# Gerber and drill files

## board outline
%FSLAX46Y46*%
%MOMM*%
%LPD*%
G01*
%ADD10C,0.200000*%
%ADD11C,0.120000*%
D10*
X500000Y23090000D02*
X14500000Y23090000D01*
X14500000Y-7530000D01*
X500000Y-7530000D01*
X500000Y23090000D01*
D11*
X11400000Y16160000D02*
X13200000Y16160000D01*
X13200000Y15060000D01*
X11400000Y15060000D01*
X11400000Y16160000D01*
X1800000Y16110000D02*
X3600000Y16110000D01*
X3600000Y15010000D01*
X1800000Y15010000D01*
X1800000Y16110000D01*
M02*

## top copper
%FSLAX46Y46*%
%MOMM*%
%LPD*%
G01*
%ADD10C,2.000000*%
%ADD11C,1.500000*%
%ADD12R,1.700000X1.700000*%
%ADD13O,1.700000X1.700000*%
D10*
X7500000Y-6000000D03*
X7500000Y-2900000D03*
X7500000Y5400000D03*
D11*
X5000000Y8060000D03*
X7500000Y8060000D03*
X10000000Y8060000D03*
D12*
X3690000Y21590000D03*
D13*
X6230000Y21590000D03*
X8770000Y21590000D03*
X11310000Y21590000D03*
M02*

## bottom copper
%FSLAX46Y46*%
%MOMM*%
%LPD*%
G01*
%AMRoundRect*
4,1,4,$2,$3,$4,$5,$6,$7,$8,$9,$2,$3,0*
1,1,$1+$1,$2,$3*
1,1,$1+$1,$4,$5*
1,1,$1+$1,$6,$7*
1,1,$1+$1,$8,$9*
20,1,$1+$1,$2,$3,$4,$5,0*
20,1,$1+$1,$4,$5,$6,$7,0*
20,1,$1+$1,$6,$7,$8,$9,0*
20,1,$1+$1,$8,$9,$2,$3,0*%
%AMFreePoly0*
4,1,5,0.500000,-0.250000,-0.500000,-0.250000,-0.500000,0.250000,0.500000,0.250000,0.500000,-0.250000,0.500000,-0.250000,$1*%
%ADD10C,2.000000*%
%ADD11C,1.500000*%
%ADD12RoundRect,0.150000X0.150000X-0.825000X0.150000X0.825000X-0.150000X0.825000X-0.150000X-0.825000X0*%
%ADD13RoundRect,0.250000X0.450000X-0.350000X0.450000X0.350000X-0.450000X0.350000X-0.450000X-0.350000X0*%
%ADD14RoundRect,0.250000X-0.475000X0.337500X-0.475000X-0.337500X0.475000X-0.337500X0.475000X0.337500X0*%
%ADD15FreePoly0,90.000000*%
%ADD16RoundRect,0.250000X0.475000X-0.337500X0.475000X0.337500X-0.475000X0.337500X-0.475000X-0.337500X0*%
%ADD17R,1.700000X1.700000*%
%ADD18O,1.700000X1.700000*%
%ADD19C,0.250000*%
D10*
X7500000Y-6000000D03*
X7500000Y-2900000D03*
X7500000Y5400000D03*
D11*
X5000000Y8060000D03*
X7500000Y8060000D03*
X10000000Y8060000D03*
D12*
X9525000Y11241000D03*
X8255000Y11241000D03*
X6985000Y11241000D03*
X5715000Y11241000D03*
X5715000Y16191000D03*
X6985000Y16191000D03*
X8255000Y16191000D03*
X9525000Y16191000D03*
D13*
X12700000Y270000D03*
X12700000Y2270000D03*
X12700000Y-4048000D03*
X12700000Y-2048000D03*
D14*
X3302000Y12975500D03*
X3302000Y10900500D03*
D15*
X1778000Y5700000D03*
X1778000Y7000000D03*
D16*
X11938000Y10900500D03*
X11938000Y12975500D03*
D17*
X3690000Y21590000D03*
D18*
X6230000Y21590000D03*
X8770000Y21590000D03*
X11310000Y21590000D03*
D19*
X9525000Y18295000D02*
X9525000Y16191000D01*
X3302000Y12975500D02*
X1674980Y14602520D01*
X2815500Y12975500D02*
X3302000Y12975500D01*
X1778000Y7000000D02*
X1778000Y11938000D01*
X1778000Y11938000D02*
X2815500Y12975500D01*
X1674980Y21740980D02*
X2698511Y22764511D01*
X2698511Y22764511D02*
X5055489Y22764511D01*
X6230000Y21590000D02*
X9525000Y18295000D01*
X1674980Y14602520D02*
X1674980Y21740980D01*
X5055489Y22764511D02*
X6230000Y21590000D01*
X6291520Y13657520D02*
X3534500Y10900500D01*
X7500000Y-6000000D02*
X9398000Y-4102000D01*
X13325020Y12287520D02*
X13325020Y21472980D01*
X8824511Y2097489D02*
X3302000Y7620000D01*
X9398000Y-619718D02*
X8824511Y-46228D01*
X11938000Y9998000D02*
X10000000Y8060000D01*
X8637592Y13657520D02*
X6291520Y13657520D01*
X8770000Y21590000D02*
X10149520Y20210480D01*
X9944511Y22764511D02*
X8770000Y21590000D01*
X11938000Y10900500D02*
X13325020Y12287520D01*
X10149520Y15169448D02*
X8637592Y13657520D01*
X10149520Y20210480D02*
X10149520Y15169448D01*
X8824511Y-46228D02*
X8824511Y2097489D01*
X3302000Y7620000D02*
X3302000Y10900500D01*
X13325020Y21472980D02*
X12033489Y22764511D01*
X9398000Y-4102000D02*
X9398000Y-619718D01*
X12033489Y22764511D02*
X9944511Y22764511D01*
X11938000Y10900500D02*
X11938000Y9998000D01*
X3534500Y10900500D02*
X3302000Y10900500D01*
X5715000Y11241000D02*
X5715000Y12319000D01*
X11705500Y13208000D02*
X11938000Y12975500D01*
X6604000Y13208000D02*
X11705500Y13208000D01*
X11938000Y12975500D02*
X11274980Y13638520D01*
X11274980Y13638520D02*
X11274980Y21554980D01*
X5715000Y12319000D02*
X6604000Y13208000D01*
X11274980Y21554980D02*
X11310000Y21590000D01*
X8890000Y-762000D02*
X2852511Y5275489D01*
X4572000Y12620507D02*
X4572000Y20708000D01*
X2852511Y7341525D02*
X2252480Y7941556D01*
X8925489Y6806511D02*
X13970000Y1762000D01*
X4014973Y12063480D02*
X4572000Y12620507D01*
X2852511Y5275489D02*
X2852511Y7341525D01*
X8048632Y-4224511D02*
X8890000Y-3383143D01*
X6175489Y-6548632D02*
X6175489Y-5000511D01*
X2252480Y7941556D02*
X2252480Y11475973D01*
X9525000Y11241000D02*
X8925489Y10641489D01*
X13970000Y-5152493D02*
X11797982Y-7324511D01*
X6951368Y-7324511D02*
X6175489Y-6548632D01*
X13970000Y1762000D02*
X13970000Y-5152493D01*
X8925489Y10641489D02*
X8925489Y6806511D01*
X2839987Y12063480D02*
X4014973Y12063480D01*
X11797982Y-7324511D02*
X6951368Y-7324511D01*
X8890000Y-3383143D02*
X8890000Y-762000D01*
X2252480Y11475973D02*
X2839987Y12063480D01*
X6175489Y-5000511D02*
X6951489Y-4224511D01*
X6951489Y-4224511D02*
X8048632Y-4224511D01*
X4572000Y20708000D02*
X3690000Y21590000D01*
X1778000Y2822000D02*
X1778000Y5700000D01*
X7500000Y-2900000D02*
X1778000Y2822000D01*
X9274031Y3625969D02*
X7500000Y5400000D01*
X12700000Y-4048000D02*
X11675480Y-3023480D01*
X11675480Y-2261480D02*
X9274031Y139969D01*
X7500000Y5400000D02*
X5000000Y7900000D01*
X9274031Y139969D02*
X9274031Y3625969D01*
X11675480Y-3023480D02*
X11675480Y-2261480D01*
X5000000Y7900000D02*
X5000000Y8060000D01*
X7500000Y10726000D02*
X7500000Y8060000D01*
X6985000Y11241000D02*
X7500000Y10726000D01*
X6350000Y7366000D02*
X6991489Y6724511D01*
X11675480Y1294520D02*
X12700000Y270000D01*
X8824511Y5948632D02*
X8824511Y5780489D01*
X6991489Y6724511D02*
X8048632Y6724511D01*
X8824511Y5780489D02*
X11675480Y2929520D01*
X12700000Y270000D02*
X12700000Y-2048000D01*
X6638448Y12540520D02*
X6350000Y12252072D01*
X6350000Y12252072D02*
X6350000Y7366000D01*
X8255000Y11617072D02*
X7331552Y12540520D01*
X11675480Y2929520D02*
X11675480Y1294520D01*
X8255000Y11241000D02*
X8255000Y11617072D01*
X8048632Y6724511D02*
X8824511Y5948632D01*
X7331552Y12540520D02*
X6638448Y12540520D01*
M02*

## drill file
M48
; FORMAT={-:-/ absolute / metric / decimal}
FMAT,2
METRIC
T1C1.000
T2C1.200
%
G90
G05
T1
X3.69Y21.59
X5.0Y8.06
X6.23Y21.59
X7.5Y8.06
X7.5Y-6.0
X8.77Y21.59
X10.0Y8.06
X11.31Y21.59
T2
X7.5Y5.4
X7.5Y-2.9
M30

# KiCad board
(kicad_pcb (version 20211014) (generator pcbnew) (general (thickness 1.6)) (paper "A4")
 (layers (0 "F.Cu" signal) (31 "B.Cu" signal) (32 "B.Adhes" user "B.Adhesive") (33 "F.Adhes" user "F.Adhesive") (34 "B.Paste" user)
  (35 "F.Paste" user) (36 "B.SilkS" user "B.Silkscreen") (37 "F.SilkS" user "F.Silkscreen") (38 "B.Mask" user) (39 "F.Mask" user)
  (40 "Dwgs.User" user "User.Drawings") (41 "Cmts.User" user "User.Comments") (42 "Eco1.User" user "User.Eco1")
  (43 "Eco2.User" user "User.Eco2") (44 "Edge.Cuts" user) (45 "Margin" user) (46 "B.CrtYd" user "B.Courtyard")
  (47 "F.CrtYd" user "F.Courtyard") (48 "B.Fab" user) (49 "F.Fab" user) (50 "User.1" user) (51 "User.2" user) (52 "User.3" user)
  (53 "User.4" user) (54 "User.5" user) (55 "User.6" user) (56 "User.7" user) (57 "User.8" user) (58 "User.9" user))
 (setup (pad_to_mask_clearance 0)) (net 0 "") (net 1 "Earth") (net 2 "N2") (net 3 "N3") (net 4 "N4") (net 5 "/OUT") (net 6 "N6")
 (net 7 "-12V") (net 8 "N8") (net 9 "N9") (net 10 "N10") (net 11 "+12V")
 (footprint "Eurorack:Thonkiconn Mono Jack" (layer "F.Cu") (at 7.5 0 90)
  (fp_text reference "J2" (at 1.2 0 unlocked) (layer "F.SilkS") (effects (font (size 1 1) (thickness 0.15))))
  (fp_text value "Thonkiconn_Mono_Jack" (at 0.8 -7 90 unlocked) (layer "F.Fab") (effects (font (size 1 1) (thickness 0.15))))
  (pad "1" thru_hole circle (at -6 0 90) (size 2 2) (drill 1) (layers *.Cu *.Mask) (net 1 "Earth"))
  (pad "2" thru_hole circle (at -2.9 0 90) (size 2 2) (drill 1.2) (layers *.Cu *.Mask) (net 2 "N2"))
  (pad "3" thru_hole circle (at 5.4 0 90) (size 2 2) (drill 1.2) (layers *.Cu *.Mask) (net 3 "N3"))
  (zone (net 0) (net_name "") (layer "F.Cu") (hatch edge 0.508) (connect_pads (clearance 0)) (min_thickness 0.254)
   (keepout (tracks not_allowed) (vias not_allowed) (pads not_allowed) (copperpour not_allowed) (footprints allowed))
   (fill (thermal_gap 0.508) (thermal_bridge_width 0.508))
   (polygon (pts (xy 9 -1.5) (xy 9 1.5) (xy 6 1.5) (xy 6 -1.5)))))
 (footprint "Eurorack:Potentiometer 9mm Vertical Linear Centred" (layer "F.Cu") (at 7.5 -15.56)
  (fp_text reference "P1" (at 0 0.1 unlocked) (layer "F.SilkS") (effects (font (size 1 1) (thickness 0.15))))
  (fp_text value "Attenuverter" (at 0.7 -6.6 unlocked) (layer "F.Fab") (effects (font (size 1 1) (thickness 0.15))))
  (fp_rect (start 3.9 0.5) (end 5.7 -0.6) (layer "Edge.Cuts") (width 0.12) (fill none))
  (fp_rect (start -5.7 0.55) (end -3.9 -0.55) (layer "Edge.Cuts") (width 0.12) (fill none))
  (pad "1" thru_hole circle (at -2.5 7.5) (size 1.5 1.5) (drill 1) (layers *.Cu *.Mask) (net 3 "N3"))
  (pad "2" thru_hole circle (at 0 7.5) (size 1.5 1.5) (drill 1) (layers *.Cu *.Mask) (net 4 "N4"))
  (pad "3" thru_hole circle (at 2.5 7.5) (size 1.5 1.5) (drill 1) (layers *.Cu *.Mask) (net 1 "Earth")))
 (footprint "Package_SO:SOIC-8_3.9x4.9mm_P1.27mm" (layer "B.Cu") (at 7.62 -13.716 90)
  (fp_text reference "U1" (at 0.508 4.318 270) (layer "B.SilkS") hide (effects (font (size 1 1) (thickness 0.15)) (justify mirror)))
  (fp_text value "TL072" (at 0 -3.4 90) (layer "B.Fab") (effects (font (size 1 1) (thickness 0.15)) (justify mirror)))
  (pad "1" smd roundrect (at -2.475 1.905 90) (size 1.95 0.6) (layers "B.Cu" "B.Paste" "B.Mask") (roundrect_rratio 0.25) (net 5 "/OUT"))
  (pad "2" smd roundrect (at -2.475 0.635 90) (size 1.95 0.6) (layers "B.Cu" "B.Paste" "B.Mask") (roundrect_rratio 0.25) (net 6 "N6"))
  (pad "3" smd roundrect (at -2.475 -0.635 90) (size 1.95 0.6) (layers "B.Cu" "B.Paste" "B.Mask") (roundrect_rratio 0.25) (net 4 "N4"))
  (pad "4" smd roundrect (at -2.475 -1.905 90) (size 1.95 0.6) (layers "B.Cu" "B.Paste" "B.Mask") (roundrect_rratio 0.25) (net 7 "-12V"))
  (pad "5" smd roundrect (at 2.475 -1.905 90) (size 1.95 0.6) (layers "B.Cu" "B.Paste" "B.Mask") (roundrect_rratio 0.25) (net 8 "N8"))
  (pad "6" smd roundrect (at 2.475 -0.635 90) (size 1.95 0.6) (layers "B.Cu" "B.Paste" "B.Mask") (roundrect_rratio 0.25) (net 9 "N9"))
  (pad "7" smd roundrect (at 2.475 0.635 90) (size 1.95 0.6) (layers "B.Cu" "B.Paste" "B.Mask") (roundrect_rratio 0.25) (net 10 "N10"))
  (pad "8" smd roundrect (at 2.475 1.905 90) (size 1.95 0.6) (layers "B.Cu" "B.Paste" "B.Mask") (roundrect_rratio 0.25) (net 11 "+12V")))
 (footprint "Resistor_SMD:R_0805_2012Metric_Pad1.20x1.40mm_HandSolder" (layer "B.Cu") (at 12.7 -1.27 90)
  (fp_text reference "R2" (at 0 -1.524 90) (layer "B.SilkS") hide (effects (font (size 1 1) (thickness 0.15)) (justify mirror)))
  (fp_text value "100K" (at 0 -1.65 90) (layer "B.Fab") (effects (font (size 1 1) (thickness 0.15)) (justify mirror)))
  (pad "1" smd roundrect (at -1 0 90) (size 1.2 1.4) (layers "B.Cu" "B.Paste" "B.Mask") (roundrect_rratio 0.208333) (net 6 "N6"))
  (pad "2" smd roundrect (at 1 0 90) (size 1.2 1.4) (layers "B.Cu" "B.Paste" "B.Mask") (roundrect_rratio 0.208333) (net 5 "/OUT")))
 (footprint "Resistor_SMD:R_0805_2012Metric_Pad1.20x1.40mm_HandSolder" (layer "B.Cu") (at 12.7 3.048 90)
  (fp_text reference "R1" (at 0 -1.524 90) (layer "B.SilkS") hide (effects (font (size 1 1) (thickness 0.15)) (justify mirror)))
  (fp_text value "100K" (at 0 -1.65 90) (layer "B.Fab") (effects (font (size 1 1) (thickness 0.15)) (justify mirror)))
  (pad "1" smd roundrect (at -1 0 90) (size 1.2 1.4) (layers "B.Cu" "B.Paste" "B.Mask") (roundrect_rratio 0.208333) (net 3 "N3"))
  (pad "2" smd roundrect (at 1 0 90) (size 1.2 1.4) (layers "B.Cu" "B.Paste" "B.Mask") (roundrect_rratio 0.208333) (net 6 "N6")))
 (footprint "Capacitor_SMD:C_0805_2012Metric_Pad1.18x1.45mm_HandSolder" (layer "B.Cu") (at 3.302 -11.938 -90)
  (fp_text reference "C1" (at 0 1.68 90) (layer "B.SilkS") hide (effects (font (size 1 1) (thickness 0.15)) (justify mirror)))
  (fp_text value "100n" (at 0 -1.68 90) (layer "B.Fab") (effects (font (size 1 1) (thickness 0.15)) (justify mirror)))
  (pad "1" smd roundrect (at -1.0375 0 270) (size 1.175 1.45) (layers "B.Cu" "B.Paste" "B.Mask") (roundrect_rratio 0.212766) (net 11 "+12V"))
  (pad "2" smd roundrect (at 1.0375 0 270) (size 1.175 1.45) (layers "B.Cu" "B.Paste" "B.Mask") (roundrect_rratio 0.212766) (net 1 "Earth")))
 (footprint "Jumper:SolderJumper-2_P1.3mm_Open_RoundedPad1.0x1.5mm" (layer "B.Cu") (at 1.778 -6.35 90)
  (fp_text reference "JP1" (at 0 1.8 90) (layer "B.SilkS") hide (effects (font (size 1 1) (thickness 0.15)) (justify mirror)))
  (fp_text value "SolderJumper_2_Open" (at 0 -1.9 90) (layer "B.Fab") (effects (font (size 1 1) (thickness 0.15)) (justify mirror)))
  (pad "1" smd custom (at -0.65 0 90) (size 1 0.5) (layers "B.Cu" "B.Mask") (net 2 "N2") (zone_connect 2)
   (options (clearance outline) (anchor rect)) (primitives))
  (pad "2" smd custom (at 0.65 0 90) (size 1 0.5) (layers "B.Cu" "B.Mask") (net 11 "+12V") (zone_connect 2)
   (options (clearance outline) (anchor rect)) (primitives)))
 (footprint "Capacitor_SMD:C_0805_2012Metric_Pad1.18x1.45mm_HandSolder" (layer "B.Cu") (at 11.938 -11.938 90)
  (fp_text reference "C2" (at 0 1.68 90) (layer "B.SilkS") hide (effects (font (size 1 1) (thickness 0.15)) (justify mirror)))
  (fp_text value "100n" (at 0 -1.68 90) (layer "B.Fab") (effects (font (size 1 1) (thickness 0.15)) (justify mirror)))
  (pad "1" smd roundrect (at -1.0375 0 90) (size 1.175 1.45) (layers "B.Cu" "B.Paste" "B.Mask") (roundrect_rratio 0.212766) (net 1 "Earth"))
  (pad "2" smd roundrect (at 1.0375 0 90) (size 1.175 1.45) (layers "B.Cu" "B.Paste" "B.Mask") (roundrect_rratio 0.212766) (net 7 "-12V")))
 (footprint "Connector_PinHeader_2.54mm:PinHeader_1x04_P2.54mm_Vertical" (layer "B.Cu") (at 3.69 -21.59 -90)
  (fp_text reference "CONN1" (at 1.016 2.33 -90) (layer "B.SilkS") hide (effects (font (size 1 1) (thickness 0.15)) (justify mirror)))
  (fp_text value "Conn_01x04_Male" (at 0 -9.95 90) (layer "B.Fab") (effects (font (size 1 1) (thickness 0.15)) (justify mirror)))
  (pad "1" thru_hole rect (at 0 0 270) (size 1.7 1.7) (drill 1) (layers *.Cu *.Mask) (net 5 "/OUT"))
  (pad "2" thru_hole oval (at 0 -2.54 270) (size 1.7 1.7) (drill 1) (layers *.Cu *.Mask) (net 11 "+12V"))
  (pad "3" thru_hole oval (at 0 -5.08 270) (size 1.7 1.7) (drill 1) (layers *.Cu *.Mask) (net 1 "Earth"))
  (pad "4" thru_hole oval (at 0 -7.62 270) (size 1.7 1.7) (drill 1) (layers *.Cu *.Mask) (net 7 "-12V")))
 (gr_rect (start 0.5 -23.09) (end 14.5 7.53) (layer "Edge.Cuts") (width 0.2) (fill none))
 (segment (start 9.525 -18.295) (end 9.525 -16.191) (width 0.25) (layer "B.Cu") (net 11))
 (segment (start 3.302 -12.9755) (end 1.67498 -14.60252) (width 0.25) (layer "B.Cu") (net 11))
 (segment (start 2.8155 -12.9755) (end 3.302 -12.9755) (width 0.25) (layer "B.Cu") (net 11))
 (segment (start 1.778 -7) (end 1.778 -11.938) (width 0.25) (layer "B.Cu") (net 11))
 (segment (start 1.778 -11.938) (end 2.8155 -12.9755) (width 0.25) (layer "B.Cu") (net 11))
 (segment (start 1.67498 -21.74098) (end 2.698511 -22.764511) (width 0.25) (layer "B.Cu") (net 11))
 (segment (start 2.698511 -22.764511) (end 5.055489 -22.764511) (width 0.25) (layer "B.Cu") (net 11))
 (segment (start 6.23 -21.59) (end 9.525 -18.295) (width 0.25) (layer "B.Cu") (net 11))
 (segment (start 1.67498 -14.60252) (end 1.67498 -21.74098) (width 0.25) (layer "B.Cu") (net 11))
 (segment (start 5.055489 -22.764511) (end 6.23 -21.59) (width 0.25) (layer "B.Cu") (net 11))
 (segment (start 6.29152 -13.65752) (end 3.5345 -10.9005) (width 0.25) (layer "B.Cu") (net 1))
 (segment (start 7.5 6) (end 9.398 4.102) (width 0.25) (layer "B.Cu") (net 1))
 (segment (start 13.32502 -12.28752) (end 13.32502 -21.47298) (width 0.25) (layer "B.Cu") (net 1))
 (segment (start 8.824511 -2.097489) (end 3.302 -7.62) (width 0.25) (layer "B.Cu") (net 1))
 (segment (start 9.398 0.619718) (end 8.824511 0.046228) (width 0.25) (layer "B.Cu") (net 1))
 (segment (start 11.938 -9.998) (end 10 -8.06) (width 0.25) (layer "B.Cu") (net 1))
 (segment (start 8.637592 -13.65752) (end 6.29152 -13.65752) (width 0.25) (layer "B.Cu") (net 1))
 (segment (start 8.77 -21.59) (end 10.14952 -20.21048) (width 0.25) (layer "B.Cu") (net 1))
 (segment (start 9.944511 -22.764511) (end 8.77 -21.59) (width 0.25) (layer "B.Cu") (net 1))
 (segment (start 11.938 -10.9005) (end 13.32502 -12.28752) (width 0.25) (layer "B.Cu") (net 1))
 (segment (start 10.14952 -15.169448) (end 8.637592 -13.65752) (width 0.25) (layer "B.Cu") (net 1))
 (segment (start 10.14952 -20.21048) (end 10.14952 -15.169448) (width 0.25) (layer "B.Cu") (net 1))
 (segment (start 8.824511 0.046228) (end 8.824511 -2.097489) (width 0.25) (layer "B.Cu") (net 1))
 (segment (start 3.302 -7.62) (end 3.302 -10.9005) (width 0.25) (layer "B.Cu") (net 1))
 (segment (start 13.32502 -21.47298) (end 12.033489 -22.764511) (width 0.25) (layer "B.Cu") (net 1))
 (segment (start 9.398 4.102) (end 9.398 0.619718) (width 0.25) (layer "B.Cu") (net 1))
 (segment (start 12.033489 -22.764511) (end 9.944511 -22.764511) (width 0.25) (layer "B.Cu") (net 1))
 (segment (start 11.938 -10.9005) (end 11.938 -9.998) (width 0.25) (layer "B.Cu") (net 1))
 (segment (start 3.5345 -10.9005) (end 3.302 -10.9005) (width 0.25) (layer "B.Cu") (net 1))
 (segment (start 5.715 -11.241) (end 5.715 -12.319) (width 0.25) (layer "B.Cu") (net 7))
 (segment (start 11.7055 -13.208) (end 11.938 -12.9755) (width 0.25) (layer "B.Cu") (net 7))
 (segment (start 6.604 -13.208) (end 11.7055 -13.208) (width 0.25) (layer "B.Cu") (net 7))
 (segment (start 11.938 -12.9755) (end 11.27498 -13.63852) (width 0.25) (layer "B.Cu") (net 7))
 (segment (start 11.27498 -13.63852) (end 11.27498 -21.55498) (width 0.25) (layer "B.Cu") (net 7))
 (segment (start 5.715 -12.319) (end 6.604 -13.208) (width 0.25) (layer "B.Cu") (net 7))
 (segment (start 11.27498 -21.55498) (end 11.31 -21.59) (width 0.25) (layer "B.Cu") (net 7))
 (segment (start 8.89 0.762) (end 2.852511 -5.275489) (width 0.25) (layer "B.Cu") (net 5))
 (segment (start 4.572 -12.620507) (end 4.572 -20.708) (width 0.25) (layer "B.Cu") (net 5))
 (segment (start 2.852511 -7.341525) (end 2.25248 -7.941556) (width 0.25) (layer "B.Cu") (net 5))
 (segment (start 8.925489 -6.806511) (end 13.97 -1.762) (width 0.25) (layer "B.Cu") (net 5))
 (segment (start 4.014973 -12.06348) (end 4.572 -12.620507) (width 0.25) (layer "B.Cu") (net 5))
 (segment (start 2.852511 -5.275489) (end 2.852511 -7.341525) (width 0.25) (layer "B.Cu") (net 5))
 (segment (start 8.048632 4.224511) (end 8.89 3.383143) (width 0.25) (layer "B.Cu") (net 5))
 (segment (start 6.175489 6.548632) (end 6.175489 5.000511) (width 0.25) (layer "B.Cu") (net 5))
 (segment (start 2.25248 -7.941556) (end 2.25248 -11.475973) (width 0.25) (layer "B.Cu") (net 5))
 (segment (start 9.525 -11.241) (end 8.925489 -10.641489) (width 0.25) (layer "B.Cu") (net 5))
 (segment (start 13.97 5.152493) (end 11.797982 7.324511) (width 0.25) (layer "B.Cu") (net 5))
 (segment (start 6.951368 7.324511) (end 6.175489 6.548632) (width 0.25) (layer "B.Cu") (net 5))
 (segment (start 13.97 -1.762) (end 13.97 5.152493) (width 0.25) (layer "B.Cu") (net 5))
 (segment (start 8.925489 -10.641489) (end 8.925489 -6.806511) (width 0.25) (layer "B.Cu") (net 5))
 (segment (start 2.839987 -12.06348) (end 4.014973 -12.06348) (width 0.25) (layer "B.Cu") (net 5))
 (segment (start 11.797982 7.324511) (end 6.951368 7.324511) (width 0.25) (layer "B.Cu") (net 5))
 (segment (start 8.89 3.383143) (end 8.89 0.762) (width 0.25) (layer "B.Cu") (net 5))
 (segment (start 2.25248 -11.475973) (end 2.839987 -12.06348) (width 0.25) (layer "B.Cu") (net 5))
 (segment (start 6.175489 5.000511) (end 6.951489 4.224511) (width 0.25) (layer "B.Cu") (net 5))
 (segment (start 6.951489 4.224511) (end 8.048632 4.224511) (width 0.25) (layer "B.Cu") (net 5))
 (segment (start 4.572 -20.708) (end 3.69 -21.59) (width 0.25) (layer "B.Cu") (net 5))
 (segment (start 1.778 -2.822) (end 1.778 -5.7) (width 0.25) (layer "B.Cu") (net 2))
 (segment (start 7.5 2.9) (end 1.778 -2.822) (width 0.25) (layer "B.Cu") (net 2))
 (segment (start 9.274031 -3.625969) (end 7.5 -5.4) (width 0.25) (layer "B.Cu") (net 3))
 (segment (start 12.7 4.048) (end 11.67548 3.02348) (width 0.25) (layer "B.Cu") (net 3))
 (segment (start 11.67548 2.26148) (end 9.274031 -0.139969) (width 0.25) (layer "B.Cu") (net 3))
 (segment (start 7.5 -5.4) (end 5 -7.9) (width 0.25) (layer "B.Cu") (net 3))
 (segment (start 9.274031 -0.139969) (end 9.274031 -3.625969) (width 0.25) (layer "B.Cu") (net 3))
 (segment (start 11.67548 3.02348) (end 11.67548 2.26148) (width 0.25) (layer "B.Cu") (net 3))
 (segment (start 5 -7.9) (end 5 -8.06) (width 0.25) (layer "B.Cu") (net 3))
 (segment (start 7.5 -10.726) (end 7.5 -8.06) (width 0.25) (layer "B.Cu") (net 4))
 (segment (start 6.985 -11.241) (end 7.5 -10.726) (width 0.25) (layer "B.Cu") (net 4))
 (segment (start 6.35 -7.366) (end 6.991489 -6.724511) (width 0.25) (layer "B.Cu") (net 6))
 (segment (start 11.67548 -1.29452) (end 12.7 -0.27) (width 0.25) (layer "B.Cu") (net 6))
 (segment (start 8.824511 -5.948632) (end 8.824511 -5.780489) (width 0.25) (layer "B.Cu") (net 6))
 (segment (start 6.991489 -6.724511) (end 8.048632 -6.724511) (width 0.25) (layer "B.Cu") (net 6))
 (segment (start 8.824511 -5.780489) (end 11.67548 -2.92952) (width 0.25) (layer "B.Cu") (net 6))
 (segment (start 12.7 -0.27) (end 12.7 2.048) (width 0.25) (layer "B.Cu") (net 6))
 (segment (start 6.638448 -12.54052) (end 6.35 -12.252072) (width 0.25) (layer "B.Cu") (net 6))
 (segment (start 6.35 -12.252072) (end 6.35 -7.366) (width 0.25) (layer "B.Cu") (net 6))
 (segment (start 8.255 -11.617072) (end 7.331552 -12.54052) (width 0.25) (layer "B.Cu") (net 6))
 (segment (start 11.67548 -2.92952) (end 11.67548 -1.29452) (width 0.25) (layer "B.Cu") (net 6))
 (segment (start 8.255 -11.241) (end 8.255 -11.617072) (width 0.25) (layer "B.Cu") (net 6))
 (segment (start 8.048632 -6.724511) (end 8.824511 -5.948632) (width 0.25) (layer "B.Cu") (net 6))
 (segment (start 7.331552 -12.54052) (end 6.638448 -12.54052) (width 0.25) (layer "B.Cu") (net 6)))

